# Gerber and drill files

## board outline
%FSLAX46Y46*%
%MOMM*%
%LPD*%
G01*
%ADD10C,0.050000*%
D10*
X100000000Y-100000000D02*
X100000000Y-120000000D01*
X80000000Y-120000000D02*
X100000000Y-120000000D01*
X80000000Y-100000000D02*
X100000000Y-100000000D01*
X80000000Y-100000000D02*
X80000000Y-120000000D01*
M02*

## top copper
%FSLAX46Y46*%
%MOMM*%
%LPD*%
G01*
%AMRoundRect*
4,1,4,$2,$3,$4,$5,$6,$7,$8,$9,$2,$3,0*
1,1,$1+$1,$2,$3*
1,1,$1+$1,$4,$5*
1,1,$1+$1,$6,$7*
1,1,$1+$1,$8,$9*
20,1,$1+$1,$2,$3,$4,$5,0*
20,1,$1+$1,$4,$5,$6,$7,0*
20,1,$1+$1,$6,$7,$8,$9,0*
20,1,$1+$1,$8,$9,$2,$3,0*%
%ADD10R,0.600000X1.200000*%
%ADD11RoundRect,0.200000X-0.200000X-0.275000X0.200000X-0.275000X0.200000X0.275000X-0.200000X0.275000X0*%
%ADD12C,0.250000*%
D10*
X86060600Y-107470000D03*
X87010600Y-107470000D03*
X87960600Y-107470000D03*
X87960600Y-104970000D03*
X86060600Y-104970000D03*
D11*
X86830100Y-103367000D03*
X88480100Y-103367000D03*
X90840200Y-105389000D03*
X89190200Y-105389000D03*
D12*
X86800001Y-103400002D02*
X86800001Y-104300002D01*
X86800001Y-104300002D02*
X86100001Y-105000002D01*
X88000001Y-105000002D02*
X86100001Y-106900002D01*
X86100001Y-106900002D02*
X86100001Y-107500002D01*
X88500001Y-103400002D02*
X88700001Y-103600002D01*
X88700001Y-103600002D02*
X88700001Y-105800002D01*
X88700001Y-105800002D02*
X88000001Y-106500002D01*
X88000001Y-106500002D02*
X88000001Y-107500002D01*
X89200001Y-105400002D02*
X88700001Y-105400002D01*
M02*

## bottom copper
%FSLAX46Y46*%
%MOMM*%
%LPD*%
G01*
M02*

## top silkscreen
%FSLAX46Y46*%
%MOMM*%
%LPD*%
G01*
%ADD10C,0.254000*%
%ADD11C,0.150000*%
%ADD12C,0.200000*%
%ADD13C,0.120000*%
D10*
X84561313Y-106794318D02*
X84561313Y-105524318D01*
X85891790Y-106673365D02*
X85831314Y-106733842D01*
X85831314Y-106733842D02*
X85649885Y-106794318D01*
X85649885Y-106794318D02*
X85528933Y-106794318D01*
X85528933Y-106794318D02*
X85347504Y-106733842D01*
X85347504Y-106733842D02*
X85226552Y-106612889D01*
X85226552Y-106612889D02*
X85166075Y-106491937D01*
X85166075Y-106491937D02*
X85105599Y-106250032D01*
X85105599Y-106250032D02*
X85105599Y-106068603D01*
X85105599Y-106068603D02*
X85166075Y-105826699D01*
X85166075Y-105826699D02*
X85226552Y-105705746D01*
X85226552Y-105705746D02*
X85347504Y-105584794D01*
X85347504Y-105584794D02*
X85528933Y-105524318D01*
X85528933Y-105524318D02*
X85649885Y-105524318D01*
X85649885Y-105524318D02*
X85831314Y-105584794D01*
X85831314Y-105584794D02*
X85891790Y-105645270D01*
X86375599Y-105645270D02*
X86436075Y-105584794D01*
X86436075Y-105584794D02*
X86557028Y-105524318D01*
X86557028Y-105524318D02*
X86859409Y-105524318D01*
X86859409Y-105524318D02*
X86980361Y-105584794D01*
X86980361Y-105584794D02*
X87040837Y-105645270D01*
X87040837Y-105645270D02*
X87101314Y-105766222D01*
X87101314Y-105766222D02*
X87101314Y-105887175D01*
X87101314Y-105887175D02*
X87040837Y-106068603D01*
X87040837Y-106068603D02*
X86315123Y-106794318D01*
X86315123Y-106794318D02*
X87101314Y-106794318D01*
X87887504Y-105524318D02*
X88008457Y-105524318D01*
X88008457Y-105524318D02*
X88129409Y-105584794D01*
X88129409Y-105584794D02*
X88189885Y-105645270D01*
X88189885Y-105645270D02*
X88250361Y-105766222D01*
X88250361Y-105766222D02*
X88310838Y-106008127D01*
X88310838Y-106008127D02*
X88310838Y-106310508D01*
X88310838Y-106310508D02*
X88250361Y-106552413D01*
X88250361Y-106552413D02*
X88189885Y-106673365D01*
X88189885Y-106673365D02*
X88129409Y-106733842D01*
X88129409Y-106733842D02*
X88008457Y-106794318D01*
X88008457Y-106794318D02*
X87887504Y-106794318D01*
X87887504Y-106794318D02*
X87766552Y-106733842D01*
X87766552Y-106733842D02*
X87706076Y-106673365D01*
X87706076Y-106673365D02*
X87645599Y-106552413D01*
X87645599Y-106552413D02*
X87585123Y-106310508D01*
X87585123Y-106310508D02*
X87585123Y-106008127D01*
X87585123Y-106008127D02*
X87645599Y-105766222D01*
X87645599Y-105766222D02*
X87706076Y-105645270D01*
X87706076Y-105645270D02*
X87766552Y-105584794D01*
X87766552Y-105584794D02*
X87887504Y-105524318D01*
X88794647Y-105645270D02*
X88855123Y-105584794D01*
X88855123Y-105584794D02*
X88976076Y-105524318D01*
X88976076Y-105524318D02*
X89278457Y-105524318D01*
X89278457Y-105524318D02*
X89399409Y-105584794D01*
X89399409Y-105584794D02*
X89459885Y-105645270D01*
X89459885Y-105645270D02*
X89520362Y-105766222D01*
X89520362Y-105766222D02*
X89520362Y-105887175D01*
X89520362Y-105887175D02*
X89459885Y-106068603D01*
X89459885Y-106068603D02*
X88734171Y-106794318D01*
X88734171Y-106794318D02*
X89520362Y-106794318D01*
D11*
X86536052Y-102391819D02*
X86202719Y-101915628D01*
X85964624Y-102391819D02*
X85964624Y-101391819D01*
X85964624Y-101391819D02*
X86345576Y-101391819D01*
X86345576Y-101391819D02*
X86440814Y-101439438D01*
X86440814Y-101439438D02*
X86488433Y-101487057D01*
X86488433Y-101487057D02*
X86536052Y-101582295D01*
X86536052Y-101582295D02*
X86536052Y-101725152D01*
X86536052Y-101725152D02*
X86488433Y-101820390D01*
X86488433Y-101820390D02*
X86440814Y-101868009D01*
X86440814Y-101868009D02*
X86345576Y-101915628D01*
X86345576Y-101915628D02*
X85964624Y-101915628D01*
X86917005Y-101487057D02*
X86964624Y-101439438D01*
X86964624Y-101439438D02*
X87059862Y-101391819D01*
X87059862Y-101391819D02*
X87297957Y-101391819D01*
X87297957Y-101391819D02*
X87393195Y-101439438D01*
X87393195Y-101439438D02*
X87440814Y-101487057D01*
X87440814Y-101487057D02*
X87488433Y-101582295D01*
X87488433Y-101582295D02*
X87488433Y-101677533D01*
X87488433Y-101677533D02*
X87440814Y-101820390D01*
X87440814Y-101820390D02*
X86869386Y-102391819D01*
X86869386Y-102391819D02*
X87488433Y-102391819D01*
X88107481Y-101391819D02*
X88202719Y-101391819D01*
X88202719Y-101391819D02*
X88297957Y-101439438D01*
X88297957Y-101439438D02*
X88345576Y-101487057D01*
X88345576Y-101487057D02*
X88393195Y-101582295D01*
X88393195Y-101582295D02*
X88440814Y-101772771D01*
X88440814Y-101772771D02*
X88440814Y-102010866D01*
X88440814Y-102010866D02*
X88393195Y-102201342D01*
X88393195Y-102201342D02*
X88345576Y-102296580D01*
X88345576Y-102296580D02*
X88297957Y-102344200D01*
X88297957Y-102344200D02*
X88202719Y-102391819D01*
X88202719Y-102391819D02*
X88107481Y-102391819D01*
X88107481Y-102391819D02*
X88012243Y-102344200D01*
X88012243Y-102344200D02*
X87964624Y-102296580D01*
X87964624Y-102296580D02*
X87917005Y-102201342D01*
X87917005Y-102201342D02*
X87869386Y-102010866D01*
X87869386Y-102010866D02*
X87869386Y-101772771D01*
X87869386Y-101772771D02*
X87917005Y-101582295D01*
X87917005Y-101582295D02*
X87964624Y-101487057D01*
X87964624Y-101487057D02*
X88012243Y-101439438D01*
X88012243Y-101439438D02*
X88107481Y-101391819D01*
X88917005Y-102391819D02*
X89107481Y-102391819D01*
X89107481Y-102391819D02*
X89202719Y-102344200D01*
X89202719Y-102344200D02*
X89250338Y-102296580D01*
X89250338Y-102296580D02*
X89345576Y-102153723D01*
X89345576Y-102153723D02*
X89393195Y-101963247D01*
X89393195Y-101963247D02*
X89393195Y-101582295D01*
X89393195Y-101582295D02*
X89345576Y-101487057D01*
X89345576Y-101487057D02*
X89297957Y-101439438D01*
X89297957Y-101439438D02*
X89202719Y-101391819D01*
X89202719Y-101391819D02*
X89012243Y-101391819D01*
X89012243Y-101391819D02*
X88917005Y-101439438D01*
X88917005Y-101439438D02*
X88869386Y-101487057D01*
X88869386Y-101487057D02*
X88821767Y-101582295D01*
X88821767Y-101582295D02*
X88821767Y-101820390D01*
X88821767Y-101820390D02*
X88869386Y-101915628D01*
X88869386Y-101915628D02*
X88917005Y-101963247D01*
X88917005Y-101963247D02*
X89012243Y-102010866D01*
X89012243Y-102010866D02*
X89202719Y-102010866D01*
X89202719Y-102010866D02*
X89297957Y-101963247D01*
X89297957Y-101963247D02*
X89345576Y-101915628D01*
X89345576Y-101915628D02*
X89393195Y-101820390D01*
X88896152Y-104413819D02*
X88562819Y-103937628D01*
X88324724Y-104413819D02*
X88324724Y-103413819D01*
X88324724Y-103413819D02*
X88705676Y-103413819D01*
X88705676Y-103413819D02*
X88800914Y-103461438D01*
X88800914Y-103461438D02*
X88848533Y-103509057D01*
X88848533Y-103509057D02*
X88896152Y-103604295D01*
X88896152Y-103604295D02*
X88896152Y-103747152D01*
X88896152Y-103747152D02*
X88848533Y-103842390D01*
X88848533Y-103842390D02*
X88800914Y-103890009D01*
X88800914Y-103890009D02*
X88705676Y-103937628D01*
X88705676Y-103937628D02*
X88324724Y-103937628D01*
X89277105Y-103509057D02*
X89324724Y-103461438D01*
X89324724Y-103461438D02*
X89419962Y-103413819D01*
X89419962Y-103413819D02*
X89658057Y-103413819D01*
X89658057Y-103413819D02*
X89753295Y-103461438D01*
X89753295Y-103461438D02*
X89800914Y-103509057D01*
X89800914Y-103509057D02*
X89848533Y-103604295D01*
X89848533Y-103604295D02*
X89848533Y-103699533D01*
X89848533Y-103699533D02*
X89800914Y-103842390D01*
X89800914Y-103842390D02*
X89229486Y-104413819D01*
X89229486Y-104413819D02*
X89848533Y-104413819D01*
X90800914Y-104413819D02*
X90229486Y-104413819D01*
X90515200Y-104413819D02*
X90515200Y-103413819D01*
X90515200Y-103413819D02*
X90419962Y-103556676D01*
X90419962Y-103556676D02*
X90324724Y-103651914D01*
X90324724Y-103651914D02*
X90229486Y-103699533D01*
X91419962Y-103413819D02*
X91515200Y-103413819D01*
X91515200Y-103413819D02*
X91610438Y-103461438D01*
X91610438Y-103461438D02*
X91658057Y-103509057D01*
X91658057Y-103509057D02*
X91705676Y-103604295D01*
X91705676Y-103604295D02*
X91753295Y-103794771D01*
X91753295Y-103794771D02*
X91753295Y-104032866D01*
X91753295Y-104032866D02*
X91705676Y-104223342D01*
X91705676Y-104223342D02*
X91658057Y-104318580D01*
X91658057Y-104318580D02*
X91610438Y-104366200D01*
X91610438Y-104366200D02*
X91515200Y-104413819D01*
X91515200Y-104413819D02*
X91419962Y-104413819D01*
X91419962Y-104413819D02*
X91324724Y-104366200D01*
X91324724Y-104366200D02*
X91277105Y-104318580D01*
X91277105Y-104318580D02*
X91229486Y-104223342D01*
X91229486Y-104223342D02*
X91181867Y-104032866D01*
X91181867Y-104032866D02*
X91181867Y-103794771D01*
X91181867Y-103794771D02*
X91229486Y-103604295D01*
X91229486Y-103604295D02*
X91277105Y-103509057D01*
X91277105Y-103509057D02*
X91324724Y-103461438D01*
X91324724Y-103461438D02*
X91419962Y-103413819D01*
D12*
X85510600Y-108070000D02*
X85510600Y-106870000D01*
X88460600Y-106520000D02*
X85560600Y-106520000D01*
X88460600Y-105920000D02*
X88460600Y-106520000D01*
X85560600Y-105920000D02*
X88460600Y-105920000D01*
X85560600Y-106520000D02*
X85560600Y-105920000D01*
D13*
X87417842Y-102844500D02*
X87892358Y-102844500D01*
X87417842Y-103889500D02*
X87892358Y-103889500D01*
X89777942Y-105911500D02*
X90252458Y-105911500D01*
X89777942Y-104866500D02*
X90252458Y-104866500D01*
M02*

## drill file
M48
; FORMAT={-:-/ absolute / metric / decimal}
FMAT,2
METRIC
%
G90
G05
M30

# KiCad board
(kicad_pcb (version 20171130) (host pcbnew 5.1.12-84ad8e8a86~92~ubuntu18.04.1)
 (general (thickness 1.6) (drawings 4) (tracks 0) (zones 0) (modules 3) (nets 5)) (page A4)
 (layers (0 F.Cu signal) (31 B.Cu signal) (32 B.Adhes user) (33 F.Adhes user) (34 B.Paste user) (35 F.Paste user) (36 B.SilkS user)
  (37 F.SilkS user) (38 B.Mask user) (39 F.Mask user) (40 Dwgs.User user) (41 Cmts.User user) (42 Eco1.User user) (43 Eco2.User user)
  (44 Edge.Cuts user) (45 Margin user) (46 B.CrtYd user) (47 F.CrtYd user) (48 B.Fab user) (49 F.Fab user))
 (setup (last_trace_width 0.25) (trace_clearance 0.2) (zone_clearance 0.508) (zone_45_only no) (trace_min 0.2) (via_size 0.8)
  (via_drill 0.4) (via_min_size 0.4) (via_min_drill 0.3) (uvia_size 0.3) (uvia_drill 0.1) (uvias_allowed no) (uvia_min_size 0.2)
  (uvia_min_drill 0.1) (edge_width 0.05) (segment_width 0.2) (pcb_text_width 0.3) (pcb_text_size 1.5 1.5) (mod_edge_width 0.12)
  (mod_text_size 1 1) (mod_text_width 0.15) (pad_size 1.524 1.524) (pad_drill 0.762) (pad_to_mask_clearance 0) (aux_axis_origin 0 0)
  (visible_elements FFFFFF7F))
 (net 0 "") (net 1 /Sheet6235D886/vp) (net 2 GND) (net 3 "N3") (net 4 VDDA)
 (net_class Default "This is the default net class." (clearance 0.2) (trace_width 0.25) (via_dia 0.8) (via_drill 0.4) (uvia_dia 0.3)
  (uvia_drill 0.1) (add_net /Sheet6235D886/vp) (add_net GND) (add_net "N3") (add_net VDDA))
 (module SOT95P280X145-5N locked (layer F.Cu) (at 87.010600 106.220000 90.000000)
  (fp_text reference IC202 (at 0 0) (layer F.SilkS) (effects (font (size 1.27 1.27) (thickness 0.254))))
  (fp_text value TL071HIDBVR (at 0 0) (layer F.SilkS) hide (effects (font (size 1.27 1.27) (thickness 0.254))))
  (fp_line (start -1.85 -1.5) (end -0.65 -1.5) (layer F.SilkS) (width 0.2))
  (fp_line (start -0.3 1.45) (end -0.3 -1.45) (layer F.SilkS) (width 0.2))
  (fp_line (start 0.3 1.45) (end -0.3 1.45) (layer F.SilkS) (width 0.2))
  (fp_line (start 0.3 -1.45) (end 0.3 1.45) (layer F.SilkS) (width 0.2))
  (fp_line (start -0.3 -1.45) (end 0.3 -1.45) (layer F.SilkS) (width 0.2))
  (pad 1 smd rect (at -1.25 -0.95 180.000000) (size 0.6 1.2) (layers F.Cu F.Mask F.Paste) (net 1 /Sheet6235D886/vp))
  (pad 2 smd rect (at -1.25 0 180.000000) (size 0.6 1.2) (layers F.Cu F.Mask F.Paste) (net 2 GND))
  (pad 3 smd rect (at -1.25 0.95 180.000000) (size 0.6 1.2) (layers F.Cu F.Mask F.Paste) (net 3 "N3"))
  (pad 4 smd rect (at 1.25 0.95 180.000000) (size 0.6 1.2) (layers F.Cu F.Mask F.Paste) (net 1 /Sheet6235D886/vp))
  (pad 5 smd rect (at 1.25 -0.95 180.000000) (size 0.6 1.2) (layers F.Cu F.Mask F.Paste) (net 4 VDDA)))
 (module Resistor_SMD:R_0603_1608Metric (layer F.Cu) (at 87.655100 103.367000)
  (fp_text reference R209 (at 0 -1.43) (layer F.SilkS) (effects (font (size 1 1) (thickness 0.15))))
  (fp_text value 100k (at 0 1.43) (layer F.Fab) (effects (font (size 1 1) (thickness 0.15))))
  (fp_line (start -0.237258 -0.5225) (end 0.237258 -0.5225) (layer F.SilkS) (width 0.12))
  (fp_line (start -0.237258 0.5225) (end 0.237258 0.5225) (layer F.SilkS) (width 0.12))
  (pad 1 smd roundrect (at -0.825 0) (size 0.8 0.95) (layers F.Cu F.Mask F.Paste) (roundrect_rratio 0.25) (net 4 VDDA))
  (pad 2 smd roundrect (at 0.825 0) (size 0.8 0.95) (layers F.Cu F.Mask F.Paste) (roundrect_rratio 0.25) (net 3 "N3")))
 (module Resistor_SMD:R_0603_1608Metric (layer F.Cu) (at 90.015200 105.389000)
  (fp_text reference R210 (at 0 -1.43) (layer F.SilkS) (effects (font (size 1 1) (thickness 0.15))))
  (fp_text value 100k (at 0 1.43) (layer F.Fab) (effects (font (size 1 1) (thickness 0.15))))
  (fp_line (start -0.237258 0.5225) (end 0.237258 0.5225) (layer F.SilkS) (width 0.12))
  (fp_line (start -0.237258 -0.5225) (end 0.237258 -0.5225) (layer F.SilkS) (width 0.12))
  (pad 2 smd roundrect (at 0.825 0) (size 0.8 0.95) (layers F.Cu F.Mask F.Paste) (roundrect_rratio 0.25) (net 2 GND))
  (pad 1 smd roundrect (at -0.825 0) (size 0.8 0.95) (layers F.Cu F.Mask F.Paste) (roundrect_rratio 0.25) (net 3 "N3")))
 (gr_line (start 100 100) (end 100 120) (layer Edge.Cuts) (width 0.05))
 (gr_line (start 80 120) (end 100 120) (layer Edge.Cuts) (width 0.05))
 (gr_line (start 80 100) (end 100 100) (layer Edge.Cuts) (width 0.05))
 (gr_line (start 80 100) (end 80 120) (layer Edge.Cuts) (width 0.05))
 (segment (start 86.800001 103.400002) (end 86.800001 104.300002) (width 0.250000) (layer F.Cu) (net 4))
 (segment (start 86.800001 104.300002) (end 86.100001 105.000002) (width 0.250000) (layer F.Cu) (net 4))
 (segment (start 88.000001 105.000002) (end 86.100001 106.900002) (width 0.250000) (layer F.Cu) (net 1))
 (segment (start 86.100001 106.900002) (end 86.100001 107.500002) (width 0.250000) (layer F.Cu) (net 1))
 (segment (start 88.500001 103.400002) (end 88.700001 103.600002) (width 0.250000) (layer F.Cu) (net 3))
 (segment (start 88.700001 103.600002) (end 88.700001 105.800002) (width 0.250000) (layer F.Cu) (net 3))
 (segment (start 88.700001 105.800002) (end 88.000001 106.500002) (width 0.250000) (layer F.Cu) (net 3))
 (segment (start 88.000001 106.500002) (end 88.000001 107.500002) (width 0.250000) (layer F.Cu) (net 3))
 (segment (start 89.200001 105.400002) (end 88.700001 105.400002) (width 0.250000) (layer F.Cu) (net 3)))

